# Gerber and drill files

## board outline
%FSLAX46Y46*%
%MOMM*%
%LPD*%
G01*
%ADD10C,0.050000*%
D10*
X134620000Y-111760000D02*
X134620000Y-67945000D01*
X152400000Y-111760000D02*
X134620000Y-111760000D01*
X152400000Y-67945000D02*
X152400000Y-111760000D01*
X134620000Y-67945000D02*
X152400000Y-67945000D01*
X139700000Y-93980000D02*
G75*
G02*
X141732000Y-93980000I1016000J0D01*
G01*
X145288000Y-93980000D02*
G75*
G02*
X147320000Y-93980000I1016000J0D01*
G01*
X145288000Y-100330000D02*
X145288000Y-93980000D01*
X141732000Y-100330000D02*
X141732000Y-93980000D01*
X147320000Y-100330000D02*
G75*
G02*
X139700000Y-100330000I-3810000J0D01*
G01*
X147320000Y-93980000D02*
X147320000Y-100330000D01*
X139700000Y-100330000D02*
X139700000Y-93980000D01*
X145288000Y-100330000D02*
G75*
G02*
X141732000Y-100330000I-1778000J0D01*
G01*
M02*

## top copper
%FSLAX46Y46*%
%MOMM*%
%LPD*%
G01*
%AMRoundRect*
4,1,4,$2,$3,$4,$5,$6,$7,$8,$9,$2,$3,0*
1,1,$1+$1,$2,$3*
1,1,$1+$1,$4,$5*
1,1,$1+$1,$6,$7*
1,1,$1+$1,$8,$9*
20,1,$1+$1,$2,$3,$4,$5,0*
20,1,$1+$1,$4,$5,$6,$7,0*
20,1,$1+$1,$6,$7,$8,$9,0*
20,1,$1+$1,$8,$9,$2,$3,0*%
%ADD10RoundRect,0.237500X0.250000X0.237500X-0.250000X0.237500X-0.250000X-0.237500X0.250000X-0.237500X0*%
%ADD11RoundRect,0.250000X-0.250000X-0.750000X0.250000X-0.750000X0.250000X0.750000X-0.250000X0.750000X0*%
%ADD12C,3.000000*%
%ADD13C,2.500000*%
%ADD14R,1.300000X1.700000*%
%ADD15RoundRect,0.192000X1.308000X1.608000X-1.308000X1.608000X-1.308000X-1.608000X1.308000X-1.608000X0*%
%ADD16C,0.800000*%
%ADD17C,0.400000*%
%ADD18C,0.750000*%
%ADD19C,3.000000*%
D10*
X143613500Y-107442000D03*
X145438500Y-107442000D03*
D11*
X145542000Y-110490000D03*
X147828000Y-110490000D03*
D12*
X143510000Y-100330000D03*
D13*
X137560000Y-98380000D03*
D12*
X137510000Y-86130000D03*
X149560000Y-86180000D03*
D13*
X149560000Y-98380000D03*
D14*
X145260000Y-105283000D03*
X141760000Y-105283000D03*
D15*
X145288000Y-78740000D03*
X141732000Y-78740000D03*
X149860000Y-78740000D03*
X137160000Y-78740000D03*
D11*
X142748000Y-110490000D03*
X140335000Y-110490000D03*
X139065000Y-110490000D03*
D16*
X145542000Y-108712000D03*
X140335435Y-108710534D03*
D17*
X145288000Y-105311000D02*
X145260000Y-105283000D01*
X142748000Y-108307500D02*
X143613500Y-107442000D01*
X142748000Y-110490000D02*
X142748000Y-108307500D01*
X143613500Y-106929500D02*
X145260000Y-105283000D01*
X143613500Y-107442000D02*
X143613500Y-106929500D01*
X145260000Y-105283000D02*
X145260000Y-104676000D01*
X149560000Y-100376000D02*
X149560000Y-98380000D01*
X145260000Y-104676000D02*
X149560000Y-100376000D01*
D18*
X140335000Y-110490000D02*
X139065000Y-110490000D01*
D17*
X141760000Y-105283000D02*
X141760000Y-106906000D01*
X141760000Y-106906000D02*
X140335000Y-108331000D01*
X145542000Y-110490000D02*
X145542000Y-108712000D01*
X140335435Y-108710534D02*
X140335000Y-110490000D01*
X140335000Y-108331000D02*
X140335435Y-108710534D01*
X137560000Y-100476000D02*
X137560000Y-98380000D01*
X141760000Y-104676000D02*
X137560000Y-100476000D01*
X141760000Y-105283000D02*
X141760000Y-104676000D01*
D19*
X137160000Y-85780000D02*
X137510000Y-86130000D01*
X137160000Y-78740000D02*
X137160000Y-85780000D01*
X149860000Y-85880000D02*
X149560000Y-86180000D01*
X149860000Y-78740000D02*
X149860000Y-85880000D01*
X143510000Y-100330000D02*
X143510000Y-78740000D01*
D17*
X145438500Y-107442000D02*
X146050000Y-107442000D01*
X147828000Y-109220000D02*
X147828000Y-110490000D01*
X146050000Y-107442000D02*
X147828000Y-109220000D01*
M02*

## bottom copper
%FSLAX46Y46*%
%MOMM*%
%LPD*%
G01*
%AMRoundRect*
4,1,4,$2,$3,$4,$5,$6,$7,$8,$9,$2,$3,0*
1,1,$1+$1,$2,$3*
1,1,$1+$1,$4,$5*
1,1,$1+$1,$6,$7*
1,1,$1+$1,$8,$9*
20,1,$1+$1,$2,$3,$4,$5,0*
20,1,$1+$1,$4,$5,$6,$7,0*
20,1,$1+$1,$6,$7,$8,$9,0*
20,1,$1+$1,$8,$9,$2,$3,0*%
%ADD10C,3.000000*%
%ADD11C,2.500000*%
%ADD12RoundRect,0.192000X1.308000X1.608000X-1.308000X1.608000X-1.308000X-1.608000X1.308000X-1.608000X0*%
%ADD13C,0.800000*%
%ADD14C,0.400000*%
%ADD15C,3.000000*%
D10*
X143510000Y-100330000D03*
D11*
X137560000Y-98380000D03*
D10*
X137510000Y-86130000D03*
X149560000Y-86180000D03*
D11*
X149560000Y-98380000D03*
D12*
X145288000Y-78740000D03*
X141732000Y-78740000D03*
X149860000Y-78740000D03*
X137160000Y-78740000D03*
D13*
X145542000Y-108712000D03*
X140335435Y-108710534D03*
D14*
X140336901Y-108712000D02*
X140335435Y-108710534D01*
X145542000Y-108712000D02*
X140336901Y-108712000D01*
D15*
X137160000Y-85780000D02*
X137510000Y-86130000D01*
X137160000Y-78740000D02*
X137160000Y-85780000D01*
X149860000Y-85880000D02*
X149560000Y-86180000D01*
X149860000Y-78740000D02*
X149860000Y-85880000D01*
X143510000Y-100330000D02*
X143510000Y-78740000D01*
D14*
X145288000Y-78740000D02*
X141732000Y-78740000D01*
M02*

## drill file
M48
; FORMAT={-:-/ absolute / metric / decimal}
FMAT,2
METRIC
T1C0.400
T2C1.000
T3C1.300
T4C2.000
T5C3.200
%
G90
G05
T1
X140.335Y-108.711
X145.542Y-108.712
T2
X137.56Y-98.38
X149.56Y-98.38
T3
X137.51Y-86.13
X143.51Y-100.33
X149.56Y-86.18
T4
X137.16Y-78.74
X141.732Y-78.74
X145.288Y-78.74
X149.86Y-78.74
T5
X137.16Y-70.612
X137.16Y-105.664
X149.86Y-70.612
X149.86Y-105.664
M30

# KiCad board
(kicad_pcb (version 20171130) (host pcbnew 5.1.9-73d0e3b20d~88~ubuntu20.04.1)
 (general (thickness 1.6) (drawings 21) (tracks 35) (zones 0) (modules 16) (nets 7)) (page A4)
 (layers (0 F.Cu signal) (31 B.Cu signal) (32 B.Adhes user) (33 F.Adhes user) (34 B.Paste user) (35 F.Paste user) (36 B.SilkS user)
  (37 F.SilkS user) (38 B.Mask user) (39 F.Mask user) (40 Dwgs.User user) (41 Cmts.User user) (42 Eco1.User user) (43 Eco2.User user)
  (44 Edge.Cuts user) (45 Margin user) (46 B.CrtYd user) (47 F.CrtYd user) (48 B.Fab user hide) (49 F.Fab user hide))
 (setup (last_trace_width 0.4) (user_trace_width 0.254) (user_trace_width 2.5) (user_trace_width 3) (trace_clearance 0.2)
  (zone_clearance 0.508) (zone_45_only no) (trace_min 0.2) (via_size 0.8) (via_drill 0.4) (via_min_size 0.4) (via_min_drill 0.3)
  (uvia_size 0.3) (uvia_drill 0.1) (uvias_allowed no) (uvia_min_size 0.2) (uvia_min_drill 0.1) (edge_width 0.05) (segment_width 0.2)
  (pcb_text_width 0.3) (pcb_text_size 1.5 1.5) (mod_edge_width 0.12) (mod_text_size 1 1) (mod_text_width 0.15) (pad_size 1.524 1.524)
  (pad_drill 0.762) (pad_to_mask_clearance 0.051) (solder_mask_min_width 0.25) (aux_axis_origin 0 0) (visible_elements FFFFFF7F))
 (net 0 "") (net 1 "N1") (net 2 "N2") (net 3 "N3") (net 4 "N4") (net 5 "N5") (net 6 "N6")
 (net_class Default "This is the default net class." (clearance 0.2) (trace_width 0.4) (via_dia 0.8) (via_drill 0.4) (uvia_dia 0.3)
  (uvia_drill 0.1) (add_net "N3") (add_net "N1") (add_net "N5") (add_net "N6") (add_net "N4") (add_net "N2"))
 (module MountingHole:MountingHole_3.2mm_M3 (layer F.Cu) (at 149.86 70.612)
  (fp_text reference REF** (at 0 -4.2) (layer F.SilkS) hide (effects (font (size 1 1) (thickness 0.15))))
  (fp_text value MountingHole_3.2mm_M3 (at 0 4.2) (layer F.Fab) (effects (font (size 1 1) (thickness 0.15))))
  (pad 1 np_thru_hole circle (at 0 0) (size 3.2 3.2) (drill 3.2) (layers *.Cu *.Mask)))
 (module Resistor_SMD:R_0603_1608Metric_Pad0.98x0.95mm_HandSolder (layer F.Cu) (at 144.526 107.442 180)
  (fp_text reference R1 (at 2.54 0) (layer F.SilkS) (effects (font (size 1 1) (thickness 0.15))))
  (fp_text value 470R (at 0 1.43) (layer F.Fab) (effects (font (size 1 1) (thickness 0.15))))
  (pad 2 smd roundrect (at 0.9125 0 180) (size 0.975 0.95) (layers F.Cu F.Paste F.Mask) (roundrect_rratio 0.25) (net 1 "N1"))
  (pad 1 smd roundrect (at -0.9125 0 180) (size 0.975 0.95) (layers F.Cu F.Paste F.Mask) (roundrect_rratio 0.25) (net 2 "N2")))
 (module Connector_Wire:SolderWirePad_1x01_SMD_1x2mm (layer F.Cu) (at 145.542 110.49)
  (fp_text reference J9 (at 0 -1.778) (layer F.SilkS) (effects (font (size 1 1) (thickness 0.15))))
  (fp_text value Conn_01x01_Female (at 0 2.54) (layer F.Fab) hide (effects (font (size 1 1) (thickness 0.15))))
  (pad 1 smd roundrect (at 0 0) (size 1 2) (layers F.Cu F.Paste F.Mask) (roundrect_rratio 0.25) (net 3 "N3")))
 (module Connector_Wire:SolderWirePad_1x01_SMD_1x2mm (layer F.Cu) (at 147.828 110.49)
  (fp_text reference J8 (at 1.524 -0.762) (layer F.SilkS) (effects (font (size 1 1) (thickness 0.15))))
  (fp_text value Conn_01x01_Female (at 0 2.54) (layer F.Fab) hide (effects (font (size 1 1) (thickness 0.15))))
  (pad 1 smd roundrect (at 0 0) (size 1 2) (layers F.Cu F.Paste F.Mask) (roundrect_rratio 0.25) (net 2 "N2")))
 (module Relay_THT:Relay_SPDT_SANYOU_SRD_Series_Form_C (layer F.Cu) (at 143.51 100.33 90)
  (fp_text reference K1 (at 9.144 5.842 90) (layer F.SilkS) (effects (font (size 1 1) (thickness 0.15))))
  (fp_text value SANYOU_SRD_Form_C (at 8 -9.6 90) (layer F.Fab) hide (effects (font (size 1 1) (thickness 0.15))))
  (pad 1 thru_hole circle (at 0 0 180) (size 3 3) (drill 1.3) (layers *.Cu *.Mask) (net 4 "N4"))
  (pad 5 thru_hole circle (at 1.95 -5.95 180) (size 2.5 2.5) (drill 1) (layers *.Cu *.Mask) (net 3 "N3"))
  (pad 4 thru_hole circle (at 14.2 -6 180) (size 3 3) (drill 1.3) (layers *.Cu *.Mask) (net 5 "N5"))
  (pad 3 thru_hole circle (at 14.15 6.05 180) (size 3 3) (drill 1.3) (layers *.Cu *.Mask) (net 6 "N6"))
  (pad 2 thru_hole circle (at 1.95 6.05 180) (size 2.5 2.5) (drill 1) (layers *.Cu *.Mask) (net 1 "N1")))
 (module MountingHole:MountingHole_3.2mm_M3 (layer F.Cu) (at 149.86 105.664)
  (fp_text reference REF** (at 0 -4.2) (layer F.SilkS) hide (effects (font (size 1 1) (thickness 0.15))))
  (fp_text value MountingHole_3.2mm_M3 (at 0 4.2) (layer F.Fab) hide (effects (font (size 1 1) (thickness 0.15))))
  (pad 1 np_thru_hole circle (at 0 0) (size 3.2 3.2) (drill 3.2) (layers *.Cu *.Mask)))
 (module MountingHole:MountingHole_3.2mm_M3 (layer F.Cu) (at 137.16 70.612)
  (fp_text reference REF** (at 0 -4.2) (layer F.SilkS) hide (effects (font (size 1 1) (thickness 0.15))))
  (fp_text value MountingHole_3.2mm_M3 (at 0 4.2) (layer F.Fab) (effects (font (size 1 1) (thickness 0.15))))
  (pad 1 np_thru_hole circle (at 0 0) (size 3.2 3.2) (drill 3.2) (layers *.Cu *.Mask)))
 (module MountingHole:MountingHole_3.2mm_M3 (layer F.Cu) (at 137.16 105.664)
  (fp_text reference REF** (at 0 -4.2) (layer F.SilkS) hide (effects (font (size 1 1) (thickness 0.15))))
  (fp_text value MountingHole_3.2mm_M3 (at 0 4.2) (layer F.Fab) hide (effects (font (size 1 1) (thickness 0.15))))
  (pad 1 np_thru_hole circle (at 0 0) (size 3.2 3.2) (drill 3.2) (layers *.Cu *.Mask)))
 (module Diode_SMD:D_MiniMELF (layer F.Cu) (at 143.51 105.283)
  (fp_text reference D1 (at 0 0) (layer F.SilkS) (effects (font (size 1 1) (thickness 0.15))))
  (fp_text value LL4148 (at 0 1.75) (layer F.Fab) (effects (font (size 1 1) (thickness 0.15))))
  (pad 2 smd rect (at 1.75 0) (size 1.3 1.7) (layers F.Cu F.Paste F.Mask) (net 1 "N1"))
  (pad 1 smd rect (at -1.75 0) (size 1.3 1.7) (layers F.Cu F.Paste F.Mask) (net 3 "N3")))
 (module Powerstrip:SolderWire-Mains (layer F.Cu) (at 145.288 78.74 180)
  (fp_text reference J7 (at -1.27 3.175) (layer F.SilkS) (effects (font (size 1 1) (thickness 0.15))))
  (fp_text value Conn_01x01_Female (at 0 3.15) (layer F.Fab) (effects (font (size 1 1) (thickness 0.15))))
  (pad 1 thru_hole roundrect (at 0 0 180) (size 3 3.6) (drill 2) (layers *.Cu *.Mask) (roundrect_rratio 0.064) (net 4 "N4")))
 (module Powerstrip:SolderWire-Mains (layer F.Cu) (at 141.732 78.74 180)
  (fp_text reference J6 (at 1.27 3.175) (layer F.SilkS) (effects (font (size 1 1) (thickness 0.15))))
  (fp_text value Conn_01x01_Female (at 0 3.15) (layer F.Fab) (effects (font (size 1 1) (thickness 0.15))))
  (pad 1 thru_hole roundrect (at 0 0 180) (size 3 3.6) (drill 2) (layers *.Cu *.Mask) (roundrect_rratio 0.064) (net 4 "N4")))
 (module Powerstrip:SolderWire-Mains (layer F.Cu) (at 149.86 78.74 180)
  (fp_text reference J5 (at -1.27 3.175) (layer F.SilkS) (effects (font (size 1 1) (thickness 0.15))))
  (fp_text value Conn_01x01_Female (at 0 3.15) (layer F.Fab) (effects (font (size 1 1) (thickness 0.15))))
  (pad 1 thru_hole roundrect (at 0 0 180) (size 3 3.6) (drill 2) (layers *.Cu *.Mask) (roundrect_rratio 0.064) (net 6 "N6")))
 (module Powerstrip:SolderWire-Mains (layer F.Cu) (at 137.16 78.74 180)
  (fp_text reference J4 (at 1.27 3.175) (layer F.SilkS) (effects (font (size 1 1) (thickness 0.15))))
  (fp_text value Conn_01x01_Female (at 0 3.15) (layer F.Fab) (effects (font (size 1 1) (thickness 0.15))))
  (pad 1 thru_hole roundrect (at 0 0 180) (size 3 3.6) (drill 2) (layers *.Cu *.Mask) (roundrect_rratio 0.064) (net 5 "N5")))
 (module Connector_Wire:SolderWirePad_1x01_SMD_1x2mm (layer F.Cu) (at 142.748 110.49)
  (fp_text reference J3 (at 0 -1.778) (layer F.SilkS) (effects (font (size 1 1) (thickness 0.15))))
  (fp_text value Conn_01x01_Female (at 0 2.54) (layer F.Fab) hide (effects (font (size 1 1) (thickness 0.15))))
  (pad 1 smd roundrect (at 0 0) (size 1 2) (layers F.Cu F.Paste F.Mask) (roundrect_rratio 0.25) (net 1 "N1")))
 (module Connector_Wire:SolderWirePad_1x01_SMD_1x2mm (layer F.Cu) (at 140.335 110.49)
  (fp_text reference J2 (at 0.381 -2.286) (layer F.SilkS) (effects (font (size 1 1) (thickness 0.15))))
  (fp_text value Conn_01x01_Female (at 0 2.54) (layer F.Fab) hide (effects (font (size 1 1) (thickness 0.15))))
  (pad 1 smd roundrect (at 0 0) (size 1 2) (layers F.Cu F.Paste F.Mask) (roundrect_rratio 0.25) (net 3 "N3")))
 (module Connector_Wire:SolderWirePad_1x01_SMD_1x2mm (layer F.Cu) (at 139.065 110.49)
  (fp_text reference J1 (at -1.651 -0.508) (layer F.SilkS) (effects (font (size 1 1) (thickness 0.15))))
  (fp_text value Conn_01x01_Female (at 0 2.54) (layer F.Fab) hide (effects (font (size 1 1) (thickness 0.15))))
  (pad 1 smd roundrect (at 0 0) (size 1 2) (layers F.Cu F.Paste F.Mask) (roundrect_rratio 0.25) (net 3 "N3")))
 (gr_line (start 134.62 111.76) (end 134.62 67.945) (layer Edge.Cuts) (width 0.05))
 (gr_line (start 152.4 111.76) (end 134.62 111.76) (layer Edge.Cuts) (width 0.05))
 (gr_line (start 152.4 67.945) (end 152.4 111.76) (layer Edge.Cuts) (width 0.05))
 (gr_line (start 134.62 67.945) (end 152.4 67.945) (layer Edge.Cuts) (width 0.05))
 (gr_arc (start 140.716 93.98) (end 141.732 93.98) (angle -180) (layer Edge.Cuts) (width 0.05))
 (gr_arc (start 146.304 93.98) (end 147.32 93.98) (angle -180) (layer Edge.Cuts) (width 0.05))
 (gr_line (start 145.288 100.33) (end 145.288 93.98) (layer Edge.Cuts) (width 0.05))
 (gr_line (start 141.732 100.33) (end 141.732 93.98) (layer Edge.Cuts) (width 0.05))
 (gr_arc (start 143.51 100.33) (end 139.7 100.33) (angle -180) (layer Edge.Cuts) (width 0.05))
 (gr_line (start 147.32 93.98) (end 147.32 100.33) (layer Edge.Cuts) (width 0.05))
 (gr_line (start 139.7 100.33) (end 139.7 93.98) (layer Edge.Cuts) (width 0.05))
 (gr_arc (start 143.51 100.33) (end 141.732 100.33) (angle -180) (layer Edge.Cuts) (width 0.05))
 (segment (start 145.288 105.311) (end 145.26 105.283) (width 0.4) (layer F.Cu) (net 1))
 (segment (start 142.748 108.3075) (end 143.6135 107.442) (width 0.4) (layer F.Cu) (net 1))
 (segment (start 142.748 110.49) (end 142.748 108.3075) (width 0.4) (layer F.Cu) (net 1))
 (segment (start 143.6135 106.9295) (end 145.26 105.283) (width 0.4) (layer F.Cu) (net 1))
 (segment (start 143.6135 107.442) (end 143.6135 106.9295) (width 0.4) (layer F.Cu) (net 1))
 (segment (start 145.26 105.283) (end 145.26 104.676) (width 0.4) (layer F.Cu) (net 1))
 (segment (start 149.56 100.376) (end 149.56 98.38) (width 0.4) (layer F.Cu) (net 1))
 (segment (start 145.26 104.676) (end 149.56 100.376) (width 0.4) (layer F.Cu) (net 1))
 (segment (start 140.335 110.49) (end 139.065 110.49) (width 0.75) (layer F.Cu) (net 3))
 (segment (start 141.76 105.283) (end 141.76 106.906) (width 0.4) (layer F.Cu) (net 3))
 (segment (start 141.76 106.906) (end 140.335 108.331) (width 0.4) (layer F.Cu) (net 3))
 (via (at 145.542 108.712) (size 0.8) (drill 0.4) (layers F.Cu B.Cu) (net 3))
 (segment (start 145.542 110.49) (end 145.542 108.712) (width 0.4) (layer F.Cu) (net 3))
 (via (at 140.335435 108.710534) (size 0.8) (drill 0.4) (layers F.Cu B.Cu) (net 3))
 (segment (start 140.336901 108.712) (end 140.335435 108.710534) (width 0.4) (layer B.Cu) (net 3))
 (segment (start 145.542 108.712) (end 140.336901 108.712) (width 0.4) (layer B.Cu) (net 3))
 (segment (start 140.335435 108.710534) (end 140.335 110.49) (width 0.4) (layer F.Cu) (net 3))
 (segment (start 140.335 108.331) (end 140.335435 108.710534) (width 0.4) (layer F.Cu) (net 3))
 (segment (start 137.56 100.476) (end 137.56 98.38) (width 0.4) (layer F.Cu) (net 3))
 (segment (start 141.76 104.676) (end 137.56 100.476) (width 0.4) (layer F.Cu) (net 3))
 (segment (start 141.76 105.283) (end 141.76 104.676) (width 0.4) (layer F.Cu) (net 3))
 (segment (start 137.16 85.78) (end 137.51 86.13) (width 3) (layer F.Cu) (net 5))
 (segment (start 137.16 78.74) (end 137.16 85.78) (width 3) (layer F.Cu) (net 5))
 (segment (start 137.16 85.78) (end 137.51 86.13) (width 3) (layer B.Cu) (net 5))
 (segment (start 137.16 78.74) (end 137.16 85.78) (width 3) (layer B.Cu) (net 5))
 (segment (start 149.86 85.88) (end 149.56 86.18) (width 3) (layer F.Cu) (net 6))
 (segment (start 149.86 78.74) (end 149.86 85.88) (width 3) (layer F.Cu) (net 6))
 (segment (start 149.86 85.88) (end 149.56 86.18) (width 3) (layer B.Cu) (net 6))
 (segment (start 149.86 78.74) (end 149.86 85.88) (width 3) (layer B.Cu) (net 6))
 (segment (start 143.51 100.33) (end 143.51 78.74) (width 3) (layer F.Cu) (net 4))
 (segment (start 143.51 100.33) (end 143.51 78.74) (width 3) (layer B.Cu) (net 4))
 (segment (start 145.288 78.74) (end 141.732 78.74) (width 0.4) (layer B.Cu) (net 4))
 (segment (start 145.4385 107.442) (end 146.05 107.442) (width 0.4) (layer F.Cu) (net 2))
 (segment (start 147.828 109.22) (end 147.828 110.49) (width 0.4) (layer F.Cu) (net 2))
 (segment (start 146.05 107.442) (end 147.828 109.22) (width 0.4) (layer F.Cu) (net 2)))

